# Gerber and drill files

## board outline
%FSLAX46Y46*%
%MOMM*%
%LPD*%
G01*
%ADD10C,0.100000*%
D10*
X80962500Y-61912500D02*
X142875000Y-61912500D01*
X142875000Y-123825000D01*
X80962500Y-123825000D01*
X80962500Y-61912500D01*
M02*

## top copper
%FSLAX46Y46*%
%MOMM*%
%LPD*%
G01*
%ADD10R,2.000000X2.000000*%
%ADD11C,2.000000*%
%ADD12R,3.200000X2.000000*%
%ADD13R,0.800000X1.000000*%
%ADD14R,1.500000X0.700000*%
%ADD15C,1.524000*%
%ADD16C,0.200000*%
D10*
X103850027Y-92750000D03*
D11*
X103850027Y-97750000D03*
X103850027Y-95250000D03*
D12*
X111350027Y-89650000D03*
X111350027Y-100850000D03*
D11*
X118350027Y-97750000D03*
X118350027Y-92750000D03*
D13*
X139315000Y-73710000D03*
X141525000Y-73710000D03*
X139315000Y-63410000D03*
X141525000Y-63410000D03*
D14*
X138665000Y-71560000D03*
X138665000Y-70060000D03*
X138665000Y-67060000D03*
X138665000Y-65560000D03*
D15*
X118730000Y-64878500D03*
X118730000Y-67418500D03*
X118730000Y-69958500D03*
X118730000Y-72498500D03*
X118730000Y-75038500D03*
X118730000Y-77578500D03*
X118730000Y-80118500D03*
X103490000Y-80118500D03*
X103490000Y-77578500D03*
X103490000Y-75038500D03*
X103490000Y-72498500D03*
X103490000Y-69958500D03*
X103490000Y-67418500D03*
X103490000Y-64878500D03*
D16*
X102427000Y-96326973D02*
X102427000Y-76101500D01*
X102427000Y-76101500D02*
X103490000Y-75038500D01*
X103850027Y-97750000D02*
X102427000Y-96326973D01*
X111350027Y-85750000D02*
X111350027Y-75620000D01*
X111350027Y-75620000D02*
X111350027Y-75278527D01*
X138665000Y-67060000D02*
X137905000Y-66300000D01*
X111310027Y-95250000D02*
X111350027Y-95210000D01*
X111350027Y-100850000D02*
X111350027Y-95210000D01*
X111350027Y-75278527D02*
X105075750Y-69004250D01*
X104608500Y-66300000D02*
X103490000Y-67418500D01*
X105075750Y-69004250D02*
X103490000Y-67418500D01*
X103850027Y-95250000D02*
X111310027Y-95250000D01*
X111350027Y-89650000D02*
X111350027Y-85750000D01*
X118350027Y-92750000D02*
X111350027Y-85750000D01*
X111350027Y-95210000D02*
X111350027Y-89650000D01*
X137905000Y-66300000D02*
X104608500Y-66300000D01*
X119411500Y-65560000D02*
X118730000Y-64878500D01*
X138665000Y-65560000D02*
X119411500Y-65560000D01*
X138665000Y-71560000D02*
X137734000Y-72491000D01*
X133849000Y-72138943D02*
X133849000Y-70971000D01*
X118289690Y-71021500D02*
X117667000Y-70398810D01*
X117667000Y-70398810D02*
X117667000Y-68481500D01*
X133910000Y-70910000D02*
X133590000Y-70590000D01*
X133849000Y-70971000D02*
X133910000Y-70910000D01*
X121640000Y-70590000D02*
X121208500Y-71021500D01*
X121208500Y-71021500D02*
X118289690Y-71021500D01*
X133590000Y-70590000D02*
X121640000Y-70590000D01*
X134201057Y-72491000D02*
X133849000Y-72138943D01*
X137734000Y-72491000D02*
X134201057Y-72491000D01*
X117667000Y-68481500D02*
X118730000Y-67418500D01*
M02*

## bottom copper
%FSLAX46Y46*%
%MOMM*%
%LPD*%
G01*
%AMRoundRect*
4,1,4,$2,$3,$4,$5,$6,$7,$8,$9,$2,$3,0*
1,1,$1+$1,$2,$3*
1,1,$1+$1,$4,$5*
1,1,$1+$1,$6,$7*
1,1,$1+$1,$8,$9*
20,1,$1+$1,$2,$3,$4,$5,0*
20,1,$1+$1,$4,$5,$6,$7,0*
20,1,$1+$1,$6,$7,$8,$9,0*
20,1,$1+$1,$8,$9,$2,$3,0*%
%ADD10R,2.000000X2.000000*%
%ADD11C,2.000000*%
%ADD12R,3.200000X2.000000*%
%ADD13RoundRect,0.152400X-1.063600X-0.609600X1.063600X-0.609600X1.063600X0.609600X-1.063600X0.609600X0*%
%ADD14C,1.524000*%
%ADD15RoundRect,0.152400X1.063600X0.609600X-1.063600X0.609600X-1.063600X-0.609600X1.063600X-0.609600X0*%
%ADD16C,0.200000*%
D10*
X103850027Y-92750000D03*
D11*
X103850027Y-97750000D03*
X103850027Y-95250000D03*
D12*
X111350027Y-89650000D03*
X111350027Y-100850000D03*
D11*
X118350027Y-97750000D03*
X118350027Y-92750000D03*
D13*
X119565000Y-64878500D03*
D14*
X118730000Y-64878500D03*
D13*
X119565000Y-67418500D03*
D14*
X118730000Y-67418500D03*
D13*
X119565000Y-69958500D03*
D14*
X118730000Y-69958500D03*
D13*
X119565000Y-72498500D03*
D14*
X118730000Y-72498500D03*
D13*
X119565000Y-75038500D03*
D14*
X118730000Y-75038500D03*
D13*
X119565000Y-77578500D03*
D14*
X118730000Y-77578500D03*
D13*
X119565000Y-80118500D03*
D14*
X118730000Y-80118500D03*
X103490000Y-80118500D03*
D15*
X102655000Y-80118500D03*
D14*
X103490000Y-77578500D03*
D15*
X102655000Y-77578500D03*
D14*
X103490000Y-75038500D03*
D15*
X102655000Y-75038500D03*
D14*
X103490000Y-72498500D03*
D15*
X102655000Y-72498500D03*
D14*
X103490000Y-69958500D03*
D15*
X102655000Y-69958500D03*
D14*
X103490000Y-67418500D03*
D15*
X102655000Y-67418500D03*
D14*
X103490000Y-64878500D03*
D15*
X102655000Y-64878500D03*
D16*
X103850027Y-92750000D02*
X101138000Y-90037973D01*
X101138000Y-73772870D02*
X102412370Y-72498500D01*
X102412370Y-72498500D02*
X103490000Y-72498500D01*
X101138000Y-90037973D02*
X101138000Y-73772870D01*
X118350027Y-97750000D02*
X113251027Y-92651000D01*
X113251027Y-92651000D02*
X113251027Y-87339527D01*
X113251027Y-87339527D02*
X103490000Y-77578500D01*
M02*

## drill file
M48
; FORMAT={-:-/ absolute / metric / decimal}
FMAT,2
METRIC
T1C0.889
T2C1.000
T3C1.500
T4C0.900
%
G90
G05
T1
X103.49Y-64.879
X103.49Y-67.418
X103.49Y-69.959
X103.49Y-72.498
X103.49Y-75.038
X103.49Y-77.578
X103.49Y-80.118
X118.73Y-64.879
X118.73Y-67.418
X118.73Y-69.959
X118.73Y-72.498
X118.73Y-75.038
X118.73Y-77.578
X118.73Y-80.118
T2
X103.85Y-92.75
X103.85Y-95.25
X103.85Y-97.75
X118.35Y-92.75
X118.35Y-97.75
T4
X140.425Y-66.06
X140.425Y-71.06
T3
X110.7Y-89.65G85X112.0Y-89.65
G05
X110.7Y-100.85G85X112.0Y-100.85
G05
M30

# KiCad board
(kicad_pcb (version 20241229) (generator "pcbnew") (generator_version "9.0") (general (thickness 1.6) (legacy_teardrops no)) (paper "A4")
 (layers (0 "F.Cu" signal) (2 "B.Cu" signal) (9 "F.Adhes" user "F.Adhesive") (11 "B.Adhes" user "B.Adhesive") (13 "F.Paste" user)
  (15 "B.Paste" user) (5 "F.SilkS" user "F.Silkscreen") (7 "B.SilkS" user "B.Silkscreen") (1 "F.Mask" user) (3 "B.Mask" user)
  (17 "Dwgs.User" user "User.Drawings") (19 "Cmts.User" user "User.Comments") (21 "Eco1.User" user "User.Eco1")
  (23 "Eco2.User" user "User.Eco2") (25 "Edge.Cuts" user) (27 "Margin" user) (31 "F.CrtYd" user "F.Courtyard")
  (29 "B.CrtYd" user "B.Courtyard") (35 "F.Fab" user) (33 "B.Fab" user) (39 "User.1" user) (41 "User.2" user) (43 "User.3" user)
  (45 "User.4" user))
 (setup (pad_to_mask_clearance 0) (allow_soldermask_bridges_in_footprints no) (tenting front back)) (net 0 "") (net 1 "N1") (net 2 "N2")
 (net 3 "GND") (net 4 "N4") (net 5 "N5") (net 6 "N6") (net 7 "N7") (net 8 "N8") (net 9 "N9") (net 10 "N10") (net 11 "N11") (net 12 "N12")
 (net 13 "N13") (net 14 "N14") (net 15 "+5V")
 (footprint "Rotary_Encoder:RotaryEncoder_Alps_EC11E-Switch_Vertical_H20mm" (layer "F.Cu") (at 103.850027 92.75)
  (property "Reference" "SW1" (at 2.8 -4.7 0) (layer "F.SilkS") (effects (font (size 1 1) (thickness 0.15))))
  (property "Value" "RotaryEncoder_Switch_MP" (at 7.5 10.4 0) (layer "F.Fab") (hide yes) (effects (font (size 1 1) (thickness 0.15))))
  (pad "A" thru_hole rect (at 0 0) (size 2 2) (drill 1) (layers "*.Cu" "*.Mask") (remove_unused_layers no) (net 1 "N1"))
  (pad "B" thru_hole circle (at 0 5) (size 2 2) (drill 1) (layers "*.Cu" "*.Mask") (remove_unused_layers no) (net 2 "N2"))
  (pad "C" thru_hole circle (at 0 2.5) (size 2 2) (drill 1) (layers "*.Cu" "*.Mask") (remove_unused_layers no) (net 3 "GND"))
  (pad "MP" thru_hole rect (at 7.5 -3.1) (size 3.2 2) (drill oval 2.8 1.5) (layers "*.Cu" "*.Mask") (remove_unused_layers no) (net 3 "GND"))
  (pad "MP" thru_hole rect (at 7.5 8.1) (size 3.2 2) (drill oval 2.8 1.5) (layers "*.Cu" "*.Mask") (remove_unused_layers no) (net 3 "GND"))
  (pad "S1" thru_hole circle (at 14.5 5) (size 2 2) (drill 1) (layers "*.Cu" "*.Mask") (remove_unused_layers no) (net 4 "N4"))
  (pad "S2" thru_hole circle (at 14.5 0) (size 2 2) (drill 1) (layers "*.Cu" "*.Mask") (remove_unused_layers no) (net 3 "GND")))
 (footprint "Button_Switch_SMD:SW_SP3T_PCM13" (layer "F.Cu") (at 140.095 68.56 90)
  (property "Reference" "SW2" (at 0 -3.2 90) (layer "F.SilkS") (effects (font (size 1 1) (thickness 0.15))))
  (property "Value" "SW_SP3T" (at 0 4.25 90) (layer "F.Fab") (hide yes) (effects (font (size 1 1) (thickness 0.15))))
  (pad "" smd rect (at -5.15 -0.78 90) (size 1 0.8) (layers "F.Cu" "F.Mask" "F.Paste"))
  (pad "" smd rect (at -5.15 1.43 90) (size 1 0.8) (layers "F.Cu" "F.Mask" "F.Paste"))
  (pad "" np_thru_hole circle (at -2.5 0.33 90) (size 0.9 0.9) (drill 0.9) (layers "*.Cu" "*.Mask"))
  (pad "" np_thru_hole circle (at 2.5 0.33 90) (size 0.9 0.9) (drill 0.9) (layers "*.Cu" "*.Mask"))
  (pad "" smd rect (at 5.15 -0.78 90) (size 1 0.8) (layers "F.Cu" "F.Mask" "F.Paste"))
  (pad "" smd rect (at 5.15 1.43 90) (size 1 0.8) (layers "F.Cu" "F.Mask" "F.Paste"))
  (pad "1" smd rect (at -3 -1.43 90) (size 0.7 1.5) (layers "F.Cu" "F.Mask" "F.Paste") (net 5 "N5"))
  (pad "2" smd rect (at -1.5 -1.43 90) (size 0.7 1.5) (layers "F.Cu" "F.Mask" "F.Paste") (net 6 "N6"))
  (pad "3" smd rect (at 1.5 -1.43 90) (size 0.7 1.5) (layers "F.Cu" "F.Mask" "F.Paste") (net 3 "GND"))
  (pad "4" smd rect (at 3 -1.43 90) (size 0.7 1.5) (layers "F.Cu" "F.Mask" "F.Paste") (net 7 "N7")))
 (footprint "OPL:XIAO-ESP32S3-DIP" (layer "B.Cu") (at 111.11 72.4985 180)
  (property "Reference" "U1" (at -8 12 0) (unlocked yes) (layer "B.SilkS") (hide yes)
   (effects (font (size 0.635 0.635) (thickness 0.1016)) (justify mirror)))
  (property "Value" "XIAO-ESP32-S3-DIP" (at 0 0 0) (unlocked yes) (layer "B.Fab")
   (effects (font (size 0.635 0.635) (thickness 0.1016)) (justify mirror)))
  (pad "1" smd roundrect (at -8.455 7.62) (size 2.432 1.524) (layers "B.Cu" "B.Mask") (roundrect_rratio 0.1) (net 7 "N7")
   (thermal_bridge_angle 45))
  (pad "1" thru_hole circle (at -7.62 7.62) (size 1.524 1.524) (drill 0.889) (layers "*.Cu" "*.Mask") (remove_unused_layers no) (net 7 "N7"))
  (pad "2" smd roundrect (at -8.455 5.08) (size 2.432 1.524) (layers "B.Cu" "B.Mask") (roundrect_rratio 0.1) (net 5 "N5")
   (thermal_bridge_angle 45))
  (pad "2" thru_hole circle (at -7.62 5.08) (size 1.524 1.524) (drill 0.889) (layers "*.Cu" "*.Mask") (remove_unused_layers no) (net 5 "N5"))
  (pad "3" smd roundrect (at -8.455 2.54) (size 2.432 1.524) (layers "B.Cu" "B.Mask") (roundrect_rratio 0.1) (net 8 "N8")
   (thermal_bridge_angle 45))
  (pad "3" thru_hole circle (at -7.62 2.54) (size 1.524 1.524) (drill 0.889) (layers "*.Cu" "*.Mask") (remove_unused_layers no) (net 8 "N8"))
  (pad "4" smd roundrect (at -8.455 0) (size 2.432 1.524) (layers "B.Cu" "B.Mask") (roundrect_rratio 0.1) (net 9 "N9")
   (thermal_bridge_angle 45))
  (pad "4" thru_hole circle (at -7.62 0) (size 1.524 1.524) (drill 0.889) (layers "*.Cu" "*.Mask") (remove_unused_layers no) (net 9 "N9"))
  (pad "5" smd roundrect (at -8.455 -2.54) (size 2.432 1.524) (layers "B.Cu" "B.Mask") (roundrect_rratio 0.1) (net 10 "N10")
   (thermal_bridge_angle 45))
  (pad "5" thru_hole circle (at -7.62 -2.54) (size 1.524 1.524) (drill 0.889) (layers "*.Cu" "*.Mask") (remove_unused_layers no)
   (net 10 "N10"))
  (pad "6" smd roundrect (at -8.455 -5.08) (size 2.432 1.524) (layers "B.Cu" "B.Mask") (roundrect_rratio 0.1) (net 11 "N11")
   (thermal_bridge_angle 45))
  (pad "6" thru_hole circle (at -7.62 -5.08) (size 1.524 1.524) (drill 0.889) (layers "*.Cu" "*.Mask") (remove_unused_layers no)
   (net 11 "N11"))
  (pad "7" smd roundrect (at -8.455 -7.62) (size 2.432 1.524) (layers "B.Cu" "B.Mask") (roundrect_rratio 0.1) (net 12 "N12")
   (thermal_bridge_angle 45))
  (pad "7" thru_hole circle (at -7.62 -7.62) (size 1.524 1.524) (drill 0.889) (layers "*.Cu" "*.Mask") (remove_unused_layers no)
   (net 12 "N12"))
  (pad "8" thru_hole circle (at 7.62 -7.62 180) (size 1.524 1.524) (drill 0.889) (layers "*.Cu" "*.Mask") (remove_unused_layers no)
   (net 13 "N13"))
  (pad "8" smd roundrect (at 8.455 -7.62 180) (size 2.432 1.524) (layers "B.Cu" "B.Mask") (roundrect_rratio 0.1) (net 13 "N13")
   (thermal_bridge_angle 45))
  (pad "9" thru_hole circle (at 7.62 -5.08 180) (size 1.524 1.524) (drill 0.889) (layers "*.Cu" "*.Mask") (remove_unused_layers no)
   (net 4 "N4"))
  (pad "9" smd roundrect (at 8.455 -5.08 180) (size 2.432 1.524) (layers "B.Cu" "B.Mask") (roundrect_rratio 0.1) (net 4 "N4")
   (thermal_bridge_angle 45))
  (pad "10" thru_hole circle (at 7.62 -2.54 180) (size 1.524 1.524) (drill 0.889) (layers "*.Cu" "*.Mask") (remove_unused_layers no)
   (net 2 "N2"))
  (pad "10" smd roundrect (at 8.455 -2.54 180) (size 2.432 1.524) (layers "B.Cu" "B.Mask") (roundrect_rratio 0.1) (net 2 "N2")
   (thermal_bridge_angle 45))
  (pad "11" thru_hole circle (at 7.62 0 180) (size 1.524 1.524) (drill 0.889) (layers "*.Cu" "*.Mask") (remove_unused_layers no)
   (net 1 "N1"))
  (pad "11" smd roundrect (at 8.455 0 180) (size 2.432 1.524) (layers "B.Cu" "B.Mask") (roundrect_rratio 0.1) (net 1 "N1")
   (thermal_bridge_angle 45))
  (pad "12" thru_hole circle (at 7.62 2.54 180) (size 1.524 1.524) (drill 0.889) (layers "*.Cu" "*.Mask") (remove_unused_layers no)
   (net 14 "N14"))
  (pad "12" smd roundrect (at 8.455 2.54 180) (size 2.432 1.524) (layers "B.Cu" "B.Mask") (roundrect_rratio 0.1) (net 14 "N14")
   (thermal_bridge_angle 45))
  (pad "13" thru_hole circle (at 7.62 5.08 180) (size 1.524 1.524) (drill 0.889) (layers "*.Cu" "*.Mask") (remove_unused_layers no)
   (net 3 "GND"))
  (pad "13" smd roundrect (at 8.455 5.08 180) (size 2.432 1.524) (layers "B.Cu" "B.Mask") (roundrect_rratio 0.1) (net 3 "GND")
   (thermal_bridge_angle 45))
  (pad "14" thru_hole circle (at 7.62 7.62 180) (size 1.524 1.524) (drill 0.889) (layers "*.Cu" "*.Mask") (remove_unused_layers no)
   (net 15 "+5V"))
  (pad "14" smd roundrect (at 8.455 7.62 180) (size 2.432 1.524) (layers "B.Cu" "B.Mask") (roundrect_rratio 0.1) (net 15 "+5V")
   (thermal_bridge_angle 45)))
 (gr_rect (start 80.9625 61.9125) (end 142.875 123.825) (stroke (width 0.1) (type solid)) (fill no) (layer "Edge.Cuts"))
 (segment (start 103.850027 92.75) (end 101.138 90.037973) (width 0.2) (layer "B.Cu") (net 1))
 (segment (start 101.138 73.77287) (end 102.41237 72.4985) (width 0.2) (layer "B.Cu") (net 1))
 (segment (start 102.41237 72.4985) (end 103.49 72.4985) (width 0.2) (layer "B.Cu") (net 1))
 (segment (start 101.138 90.037973) (end 101.138 73.77287) (width 0.2) (layer "B.Cu") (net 1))
 (segment (start 102.427 96.326973) (end 102.427 76.1015) (width 0.2) (layer "F.Cu") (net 2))
 (segment (start 102.427 76.1015) (end 103.49 75.0385) (width 0.2) (layer "F.Cu") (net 2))
 (segment (start 103.850027 97.75) (end 102.427 96.326973) (width 0.2) (layer "F.Cu") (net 2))
 (segment (start 111.350027 85.75) (end 111.350027 75.62) (width 0.2) (layer "F.Cu") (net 3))
 (segment (start 111.350027 75.62) (end 111.350027 75.278527) (width 0.2) (layer "F.Cu") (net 3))
 (segment (start 138.665 67.06) (end 137.905 66.3) (width 0.2) (layer "F.Cu") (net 3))
 (segment (start 111.310027 95.25) (end 111.350027 95.21) (width 0.2) (layer "F.Cu") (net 3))
 (segment (start 111.350027 100.85) (end 111.350027 95.21) (width 0.2) (layer "F.Cu") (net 3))
 (segment (start 111.350027 75.278527) (end 105.07575 69.00425) (width 0.2) (layer "F.Cu") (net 3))
 (segment (start 104.6085 66.3) (end 103.49 67.4185) (width 0.2) (layer "F.Cu") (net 3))
 (segment (start 105.07575 69.00425) (end 103.49 67.4185) (width 0.2) (layer "F.Cu") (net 3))
 (segment (start 103.850027 95.25) (end 111.310027 95.25) (width 0.2) (layer "F.Cu") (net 3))
 (segment (start 111.350027 89.65) (end 111.350027 85.75) (width 0.2) (layer "F.Cu") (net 3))
 (segment (start 118.350027 92.75) (end 111.350027 85.75) (width 0.2) (layer "F.Cu") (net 3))
 (segment (start 111.350027 95.21) (end 111.350027 89.65) (width 0.2) (layer "F.Cu") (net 3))
 (segment (start 137.905 66.3) (end 104.6085 66.3) (width 0.2) (layer "F.Cu") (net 3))
 (segment (start 118.350027 97.75) (end 113.251027 92.651) (width 0.2) (layer "B.Cu") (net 4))
 (segment (start 113.251027 92.651) (end 113.251027 87.339527) (width 0.2) (layer "B.Cu") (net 4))
 (segment (start 113.251027 87.339527) (end 103.49 77.5785) (width 0.2) (layer "B.Cu") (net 4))
 (segment (start 119.4115 65.56) (end 118.73 64.8785) (width 0.2) (layer "F.Cu") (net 7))
 (segment (start 138.665 65.56) (end 119.4115 65.56) (width 0.2) (layer "F.Cu") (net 7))
 (segment (start 138.665 71.56) (end 137.734 72.491) (width 0.2) (layer "F.Cu") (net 5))
 (segment (start 133.849 72.138943) (end 133.849 70.971) (width 0.2) (layer "F.Cu") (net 5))
 (segment (start 118.28969 71.0215) (end 117.667 70.39881) (width 0.2) (layer "F.Cu") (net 5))
 (segment (start 117.667 70.39881) (end 117.667 68.4815) (width 0.2) (layer "F.Cu") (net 5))
 (segment (start 133.91 70.91) (end 133.59 70.59) (width 0.2) (layer "F.Cu") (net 5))
 (segment (start 133.849 70.971) (end 133.91 70.91) (width 0.2) (layer "F.Cu") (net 5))
 (segment (start 121.64 70.59) (end 121.2085 71.0215) (width 0.2) (layer "F.Cu") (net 5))
 (segment (start 121.2085 71.0215) (end 118.28969 71.0215) (width 0.2) (layer "F.Cu") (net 5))
 (segment (start 133.59 70.59) (end 121.64 70.59) (width 0.2) (layer "F.Cu") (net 5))
 (segment (start 134.201057 72.491) (end 133.849 72.138943) (width 0.2) (layer "F.Cu") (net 5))
 (segment (start 137.734 72.491) (end 134.201057 72.491) (width 0.2) (layer "F.Cu") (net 5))
 (segment (start 117.667 68.4815) (end 118.73 67.4185) (width 0.2) (layer "F.Cu") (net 5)))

